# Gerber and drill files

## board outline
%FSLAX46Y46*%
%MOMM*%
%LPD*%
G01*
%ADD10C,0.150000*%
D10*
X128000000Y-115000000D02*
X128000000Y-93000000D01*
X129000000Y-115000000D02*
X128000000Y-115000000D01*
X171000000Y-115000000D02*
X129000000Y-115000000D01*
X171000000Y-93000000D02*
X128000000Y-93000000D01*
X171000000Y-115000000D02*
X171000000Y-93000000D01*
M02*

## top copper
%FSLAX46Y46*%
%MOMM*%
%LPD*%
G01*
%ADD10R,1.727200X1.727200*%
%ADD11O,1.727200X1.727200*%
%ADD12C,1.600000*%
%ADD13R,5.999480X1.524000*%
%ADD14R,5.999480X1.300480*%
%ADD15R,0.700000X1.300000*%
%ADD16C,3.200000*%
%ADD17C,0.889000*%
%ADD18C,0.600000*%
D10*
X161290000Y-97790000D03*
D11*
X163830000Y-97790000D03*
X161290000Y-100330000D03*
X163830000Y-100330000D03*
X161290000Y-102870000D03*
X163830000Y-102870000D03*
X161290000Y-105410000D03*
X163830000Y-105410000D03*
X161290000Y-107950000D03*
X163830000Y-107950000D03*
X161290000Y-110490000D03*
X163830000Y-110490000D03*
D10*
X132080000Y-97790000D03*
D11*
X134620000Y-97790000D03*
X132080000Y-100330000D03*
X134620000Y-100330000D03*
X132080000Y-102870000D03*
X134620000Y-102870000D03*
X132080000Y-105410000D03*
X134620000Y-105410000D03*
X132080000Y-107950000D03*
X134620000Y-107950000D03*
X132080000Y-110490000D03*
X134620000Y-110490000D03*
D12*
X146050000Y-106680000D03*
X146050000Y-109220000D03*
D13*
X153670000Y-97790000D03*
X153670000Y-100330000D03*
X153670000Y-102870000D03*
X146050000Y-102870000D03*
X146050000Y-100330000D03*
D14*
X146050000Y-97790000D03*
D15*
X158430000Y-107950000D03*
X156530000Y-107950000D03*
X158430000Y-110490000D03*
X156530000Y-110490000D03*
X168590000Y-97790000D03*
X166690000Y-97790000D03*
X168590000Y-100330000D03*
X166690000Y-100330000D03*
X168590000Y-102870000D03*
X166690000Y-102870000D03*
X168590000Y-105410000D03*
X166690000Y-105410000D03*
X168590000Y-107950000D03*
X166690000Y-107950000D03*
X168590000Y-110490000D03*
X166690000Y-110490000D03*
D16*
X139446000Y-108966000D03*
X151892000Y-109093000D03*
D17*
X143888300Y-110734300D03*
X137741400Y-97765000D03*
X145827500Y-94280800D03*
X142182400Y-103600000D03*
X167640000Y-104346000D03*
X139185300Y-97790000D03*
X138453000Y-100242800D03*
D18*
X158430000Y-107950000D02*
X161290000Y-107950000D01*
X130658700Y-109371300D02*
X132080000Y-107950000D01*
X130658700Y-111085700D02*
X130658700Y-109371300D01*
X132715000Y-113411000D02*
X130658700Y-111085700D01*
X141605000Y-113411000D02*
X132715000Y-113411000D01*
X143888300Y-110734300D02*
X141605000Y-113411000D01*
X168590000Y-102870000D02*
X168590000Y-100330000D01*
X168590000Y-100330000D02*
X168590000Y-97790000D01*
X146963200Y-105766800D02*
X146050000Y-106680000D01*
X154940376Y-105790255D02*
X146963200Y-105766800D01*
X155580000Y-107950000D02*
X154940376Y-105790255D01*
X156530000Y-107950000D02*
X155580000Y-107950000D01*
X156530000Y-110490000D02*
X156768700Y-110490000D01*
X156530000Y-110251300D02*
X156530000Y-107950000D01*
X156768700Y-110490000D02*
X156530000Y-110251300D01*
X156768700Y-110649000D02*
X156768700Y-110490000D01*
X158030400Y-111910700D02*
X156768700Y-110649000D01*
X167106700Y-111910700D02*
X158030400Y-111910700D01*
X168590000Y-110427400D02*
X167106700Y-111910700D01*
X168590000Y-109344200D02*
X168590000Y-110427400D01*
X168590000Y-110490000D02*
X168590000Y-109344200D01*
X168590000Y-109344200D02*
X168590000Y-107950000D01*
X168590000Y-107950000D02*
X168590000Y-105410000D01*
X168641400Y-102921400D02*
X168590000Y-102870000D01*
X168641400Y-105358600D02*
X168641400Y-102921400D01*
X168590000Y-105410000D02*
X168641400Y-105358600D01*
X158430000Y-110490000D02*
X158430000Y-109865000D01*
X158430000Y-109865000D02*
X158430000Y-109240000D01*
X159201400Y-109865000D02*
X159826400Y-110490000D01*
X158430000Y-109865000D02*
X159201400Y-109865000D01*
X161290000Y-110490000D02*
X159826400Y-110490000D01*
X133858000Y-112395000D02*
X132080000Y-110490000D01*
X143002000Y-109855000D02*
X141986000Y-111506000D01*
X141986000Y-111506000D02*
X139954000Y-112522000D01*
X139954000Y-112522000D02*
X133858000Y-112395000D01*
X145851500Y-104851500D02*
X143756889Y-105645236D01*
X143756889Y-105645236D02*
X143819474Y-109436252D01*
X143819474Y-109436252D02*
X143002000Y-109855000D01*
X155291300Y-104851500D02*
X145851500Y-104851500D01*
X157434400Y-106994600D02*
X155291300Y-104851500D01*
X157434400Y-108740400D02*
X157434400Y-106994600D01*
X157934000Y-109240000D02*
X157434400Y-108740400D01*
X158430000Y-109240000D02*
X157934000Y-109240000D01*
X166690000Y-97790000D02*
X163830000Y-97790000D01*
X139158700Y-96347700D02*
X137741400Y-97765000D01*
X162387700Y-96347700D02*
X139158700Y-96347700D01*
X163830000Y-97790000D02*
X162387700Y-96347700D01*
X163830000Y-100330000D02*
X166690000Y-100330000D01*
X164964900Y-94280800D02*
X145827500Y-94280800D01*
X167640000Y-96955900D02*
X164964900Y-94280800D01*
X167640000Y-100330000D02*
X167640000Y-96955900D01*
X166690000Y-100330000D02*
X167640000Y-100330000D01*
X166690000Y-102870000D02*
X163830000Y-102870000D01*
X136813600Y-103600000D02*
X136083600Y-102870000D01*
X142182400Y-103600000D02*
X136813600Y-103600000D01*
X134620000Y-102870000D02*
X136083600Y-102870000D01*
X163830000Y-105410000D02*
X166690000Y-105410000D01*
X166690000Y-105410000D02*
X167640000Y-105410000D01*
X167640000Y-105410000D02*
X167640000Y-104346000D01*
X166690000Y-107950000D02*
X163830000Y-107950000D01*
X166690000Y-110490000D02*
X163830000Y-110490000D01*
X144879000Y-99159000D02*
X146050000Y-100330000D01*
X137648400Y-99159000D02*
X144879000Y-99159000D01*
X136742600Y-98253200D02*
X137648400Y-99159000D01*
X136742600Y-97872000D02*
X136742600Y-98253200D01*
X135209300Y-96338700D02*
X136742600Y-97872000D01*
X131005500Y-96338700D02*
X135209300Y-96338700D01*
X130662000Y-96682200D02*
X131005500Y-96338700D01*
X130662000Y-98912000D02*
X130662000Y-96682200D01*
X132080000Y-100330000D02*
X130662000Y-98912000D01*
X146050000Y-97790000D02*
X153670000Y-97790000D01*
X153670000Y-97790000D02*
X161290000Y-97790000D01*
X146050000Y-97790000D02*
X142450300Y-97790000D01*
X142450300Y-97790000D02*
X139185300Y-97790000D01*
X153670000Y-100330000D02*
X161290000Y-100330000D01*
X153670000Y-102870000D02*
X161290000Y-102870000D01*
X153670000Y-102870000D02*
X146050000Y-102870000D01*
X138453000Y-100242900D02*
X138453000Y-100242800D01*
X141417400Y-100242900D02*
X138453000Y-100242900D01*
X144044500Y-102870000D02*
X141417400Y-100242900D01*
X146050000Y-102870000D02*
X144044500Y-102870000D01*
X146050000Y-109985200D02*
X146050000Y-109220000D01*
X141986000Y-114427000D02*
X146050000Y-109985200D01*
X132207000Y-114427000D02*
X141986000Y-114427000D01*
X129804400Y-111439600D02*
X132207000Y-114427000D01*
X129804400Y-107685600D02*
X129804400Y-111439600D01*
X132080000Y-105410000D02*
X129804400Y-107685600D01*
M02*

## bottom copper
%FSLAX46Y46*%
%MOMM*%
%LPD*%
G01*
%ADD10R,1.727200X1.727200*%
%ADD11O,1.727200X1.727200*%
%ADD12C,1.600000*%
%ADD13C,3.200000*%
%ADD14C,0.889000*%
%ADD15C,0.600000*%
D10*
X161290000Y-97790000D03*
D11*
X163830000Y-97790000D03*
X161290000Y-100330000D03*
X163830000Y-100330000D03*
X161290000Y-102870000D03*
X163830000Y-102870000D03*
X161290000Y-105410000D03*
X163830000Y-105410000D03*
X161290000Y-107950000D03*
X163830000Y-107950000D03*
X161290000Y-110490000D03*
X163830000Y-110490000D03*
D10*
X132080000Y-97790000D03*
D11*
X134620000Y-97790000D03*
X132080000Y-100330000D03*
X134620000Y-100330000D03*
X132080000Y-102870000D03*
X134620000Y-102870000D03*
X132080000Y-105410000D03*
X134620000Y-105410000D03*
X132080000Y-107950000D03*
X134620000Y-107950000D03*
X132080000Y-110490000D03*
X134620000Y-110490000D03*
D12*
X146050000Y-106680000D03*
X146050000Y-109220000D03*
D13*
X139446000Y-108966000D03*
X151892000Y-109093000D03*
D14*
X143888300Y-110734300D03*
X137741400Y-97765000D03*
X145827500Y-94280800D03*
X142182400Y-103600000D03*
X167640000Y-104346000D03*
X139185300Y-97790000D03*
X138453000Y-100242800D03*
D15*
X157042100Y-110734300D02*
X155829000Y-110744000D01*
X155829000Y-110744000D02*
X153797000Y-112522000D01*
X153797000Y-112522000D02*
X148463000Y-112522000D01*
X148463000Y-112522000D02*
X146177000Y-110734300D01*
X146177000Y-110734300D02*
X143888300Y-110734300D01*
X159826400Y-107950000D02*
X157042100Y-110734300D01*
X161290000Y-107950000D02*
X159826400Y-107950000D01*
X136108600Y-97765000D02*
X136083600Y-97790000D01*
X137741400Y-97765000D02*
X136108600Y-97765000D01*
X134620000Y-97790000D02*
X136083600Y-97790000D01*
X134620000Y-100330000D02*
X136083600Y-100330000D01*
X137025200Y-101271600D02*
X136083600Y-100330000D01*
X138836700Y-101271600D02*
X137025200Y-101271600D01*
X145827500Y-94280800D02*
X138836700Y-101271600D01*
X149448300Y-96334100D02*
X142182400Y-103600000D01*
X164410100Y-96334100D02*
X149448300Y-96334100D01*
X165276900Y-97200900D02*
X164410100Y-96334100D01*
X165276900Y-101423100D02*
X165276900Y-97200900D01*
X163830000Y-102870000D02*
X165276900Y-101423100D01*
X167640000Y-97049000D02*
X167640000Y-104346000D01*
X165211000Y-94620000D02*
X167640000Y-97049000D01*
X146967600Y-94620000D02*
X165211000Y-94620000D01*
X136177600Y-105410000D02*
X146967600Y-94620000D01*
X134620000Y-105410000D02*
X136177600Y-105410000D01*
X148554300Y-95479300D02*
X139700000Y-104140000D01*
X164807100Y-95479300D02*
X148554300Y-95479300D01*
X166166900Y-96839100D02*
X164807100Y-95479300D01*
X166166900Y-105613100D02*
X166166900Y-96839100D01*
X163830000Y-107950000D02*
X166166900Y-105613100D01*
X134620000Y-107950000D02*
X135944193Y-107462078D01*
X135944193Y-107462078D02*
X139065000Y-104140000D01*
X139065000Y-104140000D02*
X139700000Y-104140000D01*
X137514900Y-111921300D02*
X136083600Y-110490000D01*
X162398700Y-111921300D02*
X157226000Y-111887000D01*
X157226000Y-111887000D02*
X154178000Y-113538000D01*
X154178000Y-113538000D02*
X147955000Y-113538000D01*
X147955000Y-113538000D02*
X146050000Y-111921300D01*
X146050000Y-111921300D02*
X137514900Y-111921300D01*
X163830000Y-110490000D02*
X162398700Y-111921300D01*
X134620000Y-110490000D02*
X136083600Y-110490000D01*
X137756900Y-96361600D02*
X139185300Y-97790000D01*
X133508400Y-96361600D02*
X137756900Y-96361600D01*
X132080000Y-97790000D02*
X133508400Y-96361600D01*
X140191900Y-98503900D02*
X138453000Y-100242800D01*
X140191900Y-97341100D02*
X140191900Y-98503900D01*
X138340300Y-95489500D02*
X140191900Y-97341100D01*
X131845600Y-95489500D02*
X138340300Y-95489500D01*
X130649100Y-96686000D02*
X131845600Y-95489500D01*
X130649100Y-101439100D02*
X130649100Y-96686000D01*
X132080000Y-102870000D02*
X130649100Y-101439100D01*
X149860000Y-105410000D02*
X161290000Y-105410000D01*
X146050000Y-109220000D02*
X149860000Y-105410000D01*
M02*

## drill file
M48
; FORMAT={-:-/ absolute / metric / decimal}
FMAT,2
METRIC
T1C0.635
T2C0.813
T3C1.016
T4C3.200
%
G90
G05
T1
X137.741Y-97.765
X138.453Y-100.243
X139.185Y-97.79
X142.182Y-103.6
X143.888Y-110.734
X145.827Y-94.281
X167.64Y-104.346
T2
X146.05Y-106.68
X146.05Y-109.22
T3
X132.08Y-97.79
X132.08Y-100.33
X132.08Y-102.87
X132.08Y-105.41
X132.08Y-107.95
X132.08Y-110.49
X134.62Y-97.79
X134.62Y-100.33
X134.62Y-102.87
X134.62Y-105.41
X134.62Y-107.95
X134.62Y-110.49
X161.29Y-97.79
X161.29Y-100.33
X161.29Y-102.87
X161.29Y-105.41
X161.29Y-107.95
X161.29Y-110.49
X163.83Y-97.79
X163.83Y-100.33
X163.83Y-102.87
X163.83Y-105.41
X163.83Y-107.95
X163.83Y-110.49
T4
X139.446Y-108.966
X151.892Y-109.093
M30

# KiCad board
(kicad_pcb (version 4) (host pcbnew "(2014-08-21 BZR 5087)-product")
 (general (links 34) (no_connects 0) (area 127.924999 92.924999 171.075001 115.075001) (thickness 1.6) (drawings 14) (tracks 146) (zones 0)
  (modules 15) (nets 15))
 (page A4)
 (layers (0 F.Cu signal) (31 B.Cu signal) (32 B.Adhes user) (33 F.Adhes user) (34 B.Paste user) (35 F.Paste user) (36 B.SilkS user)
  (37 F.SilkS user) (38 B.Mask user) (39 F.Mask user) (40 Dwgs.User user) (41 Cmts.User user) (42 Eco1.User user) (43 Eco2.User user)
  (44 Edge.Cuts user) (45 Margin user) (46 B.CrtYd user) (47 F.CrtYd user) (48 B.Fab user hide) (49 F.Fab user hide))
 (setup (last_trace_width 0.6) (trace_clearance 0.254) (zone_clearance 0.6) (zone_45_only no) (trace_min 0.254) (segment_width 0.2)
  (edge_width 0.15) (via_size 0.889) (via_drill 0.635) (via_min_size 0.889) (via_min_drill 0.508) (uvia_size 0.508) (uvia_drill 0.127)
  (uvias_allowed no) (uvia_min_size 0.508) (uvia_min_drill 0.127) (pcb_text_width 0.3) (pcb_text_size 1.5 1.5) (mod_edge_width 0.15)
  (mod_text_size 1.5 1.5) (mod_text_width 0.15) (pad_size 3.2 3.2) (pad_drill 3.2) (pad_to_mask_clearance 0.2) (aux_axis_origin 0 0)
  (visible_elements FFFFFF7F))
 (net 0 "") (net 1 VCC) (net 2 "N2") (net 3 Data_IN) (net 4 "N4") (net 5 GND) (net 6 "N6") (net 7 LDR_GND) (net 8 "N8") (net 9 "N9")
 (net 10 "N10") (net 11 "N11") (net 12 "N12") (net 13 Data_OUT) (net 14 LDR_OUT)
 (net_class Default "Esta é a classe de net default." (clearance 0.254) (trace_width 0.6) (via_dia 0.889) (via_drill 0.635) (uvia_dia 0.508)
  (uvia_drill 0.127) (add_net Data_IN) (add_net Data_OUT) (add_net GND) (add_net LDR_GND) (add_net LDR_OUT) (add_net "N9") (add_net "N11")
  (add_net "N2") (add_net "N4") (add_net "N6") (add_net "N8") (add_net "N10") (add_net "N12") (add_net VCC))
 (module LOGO (layer F.Cu) (at 0 0)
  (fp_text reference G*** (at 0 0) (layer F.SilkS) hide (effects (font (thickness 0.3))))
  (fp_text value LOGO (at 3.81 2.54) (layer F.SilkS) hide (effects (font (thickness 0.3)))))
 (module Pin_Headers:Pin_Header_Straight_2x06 (layer F.Cu) (at 161.29 97.79)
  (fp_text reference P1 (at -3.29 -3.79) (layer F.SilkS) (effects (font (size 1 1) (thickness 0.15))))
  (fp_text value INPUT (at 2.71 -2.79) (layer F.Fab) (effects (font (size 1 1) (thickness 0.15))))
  (pad 1 thru_hole rect (at 0 0) (size 1.7272 1.7272) (drill 1.016) (layers *.Cu *.Mask F.SilkS) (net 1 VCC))
  (pad 2 thru_hole oval (at 2.54 0) (size 1.7272 1.7272) (drill 1.016) (layers *.Cu *.Mask F.SilkS) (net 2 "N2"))
  (pad 3 thru_hole oval (at 0 2.54) (size 1.7272 1.7272) (drill 1.016) (layers *.Cu *.Mask F.SilkS) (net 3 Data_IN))
  (pad 4 thru_hole oval (at 2.54 2.54) (size 1.7272 1.7272) (drill 1.016) (layers *.Cu *.Mask F.SilkS) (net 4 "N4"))
  (pad 5 thru_hole oval (at 0 5.08) (size 1.7272 1.7272) (drill 1.016) (layers *.Cu *.Mask F.SilkS) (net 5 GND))
  (pad 6 thru_hole oval (at 2.54 5.08) (size 1.7272 1.7272) (drill 1.016) (layers *.Cu *.Mask F.SilkS) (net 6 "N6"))
  (pad 7 thru_hole oval (at 0 7.62) (size 1.7272 1.7272) (drill 1.016) (layers *.Cu *.Mask F.SilkS) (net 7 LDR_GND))
  (pad 8 thru_hole oval (at 2.54 7.62) (size 1.7272 1.7272) (drill 1.016) (layers *.Cu *.Mask F.SilkS) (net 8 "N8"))
  (pad 9 thru_hole oval (at 0 10.16) (size 1.7272 1.7272) (drill 1.016) (layers *.Cu *.Mask F.SilkS) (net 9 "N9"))
  (pad 10 thru_hole oval (at 2.54 10.16) (size 1.7272 1.7272) (drill 1.016) (layers *.Cu *.Mask F.SilkS) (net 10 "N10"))
  (pad 11 thru_hole oval (at 0 12.7) (size 1.7272 1.7272) (drill 1.016) (layers *.Cu *.Mask F.SilkS) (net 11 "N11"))
  (pad 12 thru_hole oval (at 2.54 12.7) (size 1.7272 1.7272) (drill 1.016) (layers *.Cu *.Mask F.SilkS) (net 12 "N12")))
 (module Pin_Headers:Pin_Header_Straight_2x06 (layer F.Cu) (at 132.08 97.79)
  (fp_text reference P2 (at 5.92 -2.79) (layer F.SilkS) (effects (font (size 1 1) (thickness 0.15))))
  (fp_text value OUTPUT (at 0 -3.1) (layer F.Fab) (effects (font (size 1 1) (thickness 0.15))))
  (pad 1 thru_hole rect (at 0 0) (size 1.7272 1.7272) (drill 1.016) (layers *.Cu *.Mask F.SilkS) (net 1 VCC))
  (pad 2 thru_hole oval (at 2.54 0) (size 1.7272 1.7272) (drill 1.016) (layers *.Cu *.Mask F.SilkS) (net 2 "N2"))
  (pad 3 thru_hole oval (at 0 2.54) (size 1.7272 1.7272) (drill 1.016) (layers *.Cu *.Mask F.SilkS) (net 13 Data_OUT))
  (pad 4 thru_hole oval (at 2.54 2.54) (size 1.7272 1.7272) (drill 1.016) (layers *.Cu *.Mask F.SilkS) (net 4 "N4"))
  (pad 5 thru_hole oval (at 0 5.08) (size 1.7272 1.7272) (drill 1.016) (layers *.Cu *.Mask F.SilkS) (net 5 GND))
  (pad 6 thru_hole oval (at 2.54 5.08) (size 1.7272 1.7272) (drill 1.016) (layers *.Cu *.Mask F.SilkS) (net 6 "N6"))
  (pad 7 thru_hole oval (at 0 7.62) (size 1.7272 1.7272) (drill 1.016) (layers *.Cu *.Mask F.SilkS) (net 7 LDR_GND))
  (pad 8 thru_hole oval (at 2.54 7.62) (size 1.7272 1.7272) (drill 1.016) (layers *.Cu *.Mask F.SilkS) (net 8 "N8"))
  (pad 9 thru_hole oval (at 0 10.16) (size 1.7272 1.7272) (drill 1.016) (layers *.Cu *.Mask F.SilkS) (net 9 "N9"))
  (pad 10 thru_hole oval (at 2.54 10.16) (size 1.7272 1.7272) (drill 1.016) (layers *.Cu *.Mask F.SilkS) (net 10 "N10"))
  (pad 11 thru_hole oval (at 0 12.7) (size 1.7272 1.7272) (drill 1.016) (layers *.Cu *.Mask F.SilkS) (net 11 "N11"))
  (pad 12 thru_hole oval (at 2.54 12.7) (size 1.7272 1.7272) (drill 1.016) (layers *.Cu *.Mask F.SilkS) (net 12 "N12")))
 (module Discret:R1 (layer F.Cu) (at 146.05 107.95 270)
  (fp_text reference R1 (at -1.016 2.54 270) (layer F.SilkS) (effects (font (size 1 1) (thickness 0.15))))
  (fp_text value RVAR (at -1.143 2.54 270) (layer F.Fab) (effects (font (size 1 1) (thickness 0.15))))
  (pad 1 thru_hole circle (at -1.27 0 270) (size 1.6 1.6) (drill 0.8128) (layers *.Cu *.Mask F.SilkS) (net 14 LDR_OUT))
  (pad 2 thru_hole circle (at 1.27 0 270) (size 1.6 1.6) (drill 0.8128) (layers *.Cu *.Mask F.SilkS) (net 7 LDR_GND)))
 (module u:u (layer F.Cu) (at 149.86 100.33)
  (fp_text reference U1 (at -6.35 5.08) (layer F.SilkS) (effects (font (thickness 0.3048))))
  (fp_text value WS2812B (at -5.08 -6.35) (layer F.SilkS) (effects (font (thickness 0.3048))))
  (pad 1 smd rect (at 3.81 -2.54) (size 5.99948 1.524) (layers F.Cu F.Paste F.Mask) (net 1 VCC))
  (pad 2 smd rect (at 3.81 0) (size 5.99948 1.524) (layers F.Cu F.Paste F.Mask) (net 3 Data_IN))
  (pad 3 smd rect (at 3.81 2.54) (size 5.99948 1.524) (layers F.Cu F.Paste F.Mask) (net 5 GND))
  (pad 4 smd rect (at -3.81 2.54) (size 5.99948 1.524) (layers F.Cu F.Paste F.Mask) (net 5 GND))
  (pad 5 smd rect (at -3.81 0) (size 5.99948 1.524) (layers F.Cu F.Paste F.Mask) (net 13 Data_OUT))
  (pad 6 smd rect (at -3.81 -2.54) (size 5.99948 1.30048) (layers F.Cu F.Paste F.Mask) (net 1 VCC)))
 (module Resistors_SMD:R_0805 (layer F.Cu) (at 157.48 107.95 180)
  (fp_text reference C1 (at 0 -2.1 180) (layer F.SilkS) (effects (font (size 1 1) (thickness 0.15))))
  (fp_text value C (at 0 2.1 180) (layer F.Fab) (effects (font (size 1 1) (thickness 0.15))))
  (pad 1 smd rect (at -0.95 0 180) (size 0.7 1.3) (layers F.Cu F.Paste F.Mask) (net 9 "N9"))
  (pad 2 smd rect (at 0.95 0 180) (size 0.7 1.3) (layers F.Cu F.Paste F.Mask) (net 14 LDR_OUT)))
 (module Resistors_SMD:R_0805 (layer F.Cu) (at 157.48 110.49 180)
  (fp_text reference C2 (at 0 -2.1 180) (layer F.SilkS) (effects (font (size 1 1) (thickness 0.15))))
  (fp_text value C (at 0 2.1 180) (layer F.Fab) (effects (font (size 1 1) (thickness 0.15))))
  (pad 1 smd rect (at -0.95 0 180) (size 0.7 1.3) (layers F.Cu F.Paste F.Mask) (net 11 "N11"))
  (pad 2 smd rect (at 0.95 0 180) (size 0.7 1.3) (layers F.Cu F.Paste F.Mask) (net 14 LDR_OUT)))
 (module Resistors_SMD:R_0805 (layer F.Cu) (at 167.64 97.79 180)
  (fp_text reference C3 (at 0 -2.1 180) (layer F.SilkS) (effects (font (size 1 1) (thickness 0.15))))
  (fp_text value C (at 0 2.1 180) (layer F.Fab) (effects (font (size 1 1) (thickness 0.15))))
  (pad 1 smd rect (at -0.95 0 180) (size 0.7 1.3) (layers F.Cu F.Paste F.Mask) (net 14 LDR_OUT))
  (pad 2 smd rect (at 0.95 0 180) (size 0.7 1.3) (layers F.Cu F.Paste F.Mask) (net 2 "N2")))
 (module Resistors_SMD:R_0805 (layer F.Cu) (at 167.64 100.33 180)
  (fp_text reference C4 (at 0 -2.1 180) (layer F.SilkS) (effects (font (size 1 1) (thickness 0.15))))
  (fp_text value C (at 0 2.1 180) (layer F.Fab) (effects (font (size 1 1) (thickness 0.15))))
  (pad 1 smd rect (at -0.95 0 180) (size 0.7 1.3) (layers F.Cu F.Paste F.Mask) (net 14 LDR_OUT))
  (pad 2 smd rect (at 0.95 0 180) (size 0.7 1.3) (layers F.Cu F.Paste F.Mask) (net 4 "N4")))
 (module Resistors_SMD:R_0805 (layer F.Cu) (at 167.64 102.87 180)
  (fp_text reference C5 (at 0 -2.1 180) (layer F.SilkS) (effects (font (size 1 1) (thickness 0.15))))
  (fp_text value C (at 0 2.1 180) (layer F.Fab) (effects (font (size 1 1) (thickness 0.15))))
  (pad 1 smd rect (at -0.95 0 180) (size 0.7 1.3) (layers F.Cu F.Paste F.Mask) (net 14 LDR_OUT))
  (pad 2 smd rect (at 0.95 0 180) (size 0.7 1.3) (layers F.Cu F.Paste F.Mask) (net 6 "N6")))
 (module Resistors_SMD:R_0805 (layer F.Cu) (at 167.64 105.41 180)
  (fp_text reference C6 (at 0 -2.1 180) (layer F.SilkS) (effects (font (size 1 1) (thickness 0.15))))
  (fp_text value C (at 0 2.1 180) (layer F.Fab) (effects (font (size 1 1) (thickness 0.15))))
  (pad 1 smd rect (at -0.95 0 180) (size 0.7 1.3) (layers F.Cu F.Paste F.Mask) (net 14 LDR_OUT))
  (pad 2 smd rect (at 0.95 0 180) (size 0.7 1.3) (layers F.Cu F.Paste F.Mask) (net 8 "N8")))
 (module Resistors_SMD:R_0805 (layer F.Cu) (at 167.64 107.95 180)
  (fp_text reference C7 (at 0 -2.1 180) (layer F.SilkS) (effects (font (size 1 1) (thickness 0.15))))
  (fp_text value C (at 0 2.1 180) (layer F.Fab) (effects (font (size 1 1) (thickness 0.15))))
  (pad 1 smd rect (at -0.95 0 180) (size 0.7 1.3) (layers F.Cu F.Paste F.Mask) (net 14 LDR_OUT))
  (pad 2 smd rect (at 0.95 0 180) (size 0.7 1.3) (layers F.Cu F.Paste F.Mask) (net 10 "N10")))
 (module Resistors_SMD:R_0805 (layer F.Cu) (at 167.64 110.49 180)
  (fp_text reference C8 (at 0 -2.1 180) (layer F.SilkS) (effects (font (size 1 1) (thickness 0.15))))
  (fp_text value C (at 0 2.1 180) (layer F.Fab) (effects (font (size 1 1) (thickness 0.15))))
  (pad 1 smd rect (at -0.95 0 180) (size 0.7 1.3) (layers F.Cu F.Paste F.Mask) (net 14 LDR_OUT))
  (pad 2 smd rect (at 0.95 0 180) (size 0.7 1.3) (layers F.Cu F.Paste F.Mask) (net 12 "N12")))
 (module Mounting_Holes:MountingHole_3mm (layer F.Cu) (at 139.446 108.966)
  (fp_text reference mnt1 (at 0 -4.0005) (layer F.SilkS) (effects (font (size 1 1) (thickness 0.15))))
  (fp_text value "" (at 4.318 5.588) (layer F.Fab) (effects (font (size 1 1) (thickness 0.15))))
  (pad "" thru_hole circle (at 0 0) (size 3.2 3.2) (drill 3.2) (layers *.Cu *.Mask F.SilkS)))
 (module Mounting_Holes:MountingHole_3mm (layer F.Cu) (at 151.892 109.093)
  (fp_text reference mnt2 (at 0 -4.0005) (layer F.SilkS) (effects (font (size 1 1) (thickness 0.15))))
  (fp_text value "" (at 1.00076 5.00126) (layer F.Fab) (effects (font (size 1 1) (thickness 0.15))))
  (pad "" thru_hole circle (at 0 0) (size 3.2 3.2) (drill 3.2) (layers *.Cu)))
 (gr_line (start 128 115) (end 128 93) (angle 90) (layer Edge.Cuts) (width 0.15))
 (gr_line (start 129 115) (end 128 115) (angle 90) (layer Edge.Cuts) (width 0.15))
 (gr_line (start 171 115) (end 129 115) (angle 90) (layer Edge.Cuts) (width 0.15))
 (gr_line (start 171 93) (end 128 93) (angle 90) (layer Edge.Cuts) (width 0.15))
 (gr_line (start 171 115) (end 171 93) (angle 90) (layer Edge.Cuts) (width 0.15))
 (via (at 143.8883 110.7343) (size 0.889) (layers F.Cu B.Cu) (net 9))
 (segment (start 158.43 107.95) (end 161.29 107.95) (width 0.6) (layer F.Cu) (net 9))
 (segment (start 157.0421 110.7343) (end 155.829 110.744) (width 0.6) (layer B.Cu) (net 9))
 (segment (start 155.829 110.744) (end 153.797 112.522) (width 0.6) (layer B.Cu) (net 9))
 (segment (start 153.797 112.522) (end 148.463 112.522) (width 0.6) (layer B.Cu) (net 9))
 (segment (start 148.463 112.522) (end 146.177 110.7343) (width 0.6) (layer B.Cu) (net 9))
 (segment (start 146.177 110.7343) (end 143.8883 110.7343) (width 0.6) (layer B.Cu) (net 9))
 (segment (start 159.8264 107.95) (end 157.0421 110.7343) (width 0.6) (layer B.Cu) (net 9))
 (segment (start 130.6587 109.3713) (end 132.08 107.95) (width 0.6) (layer F.Cu) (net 9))
 (segment (start 130.6587 111.0857) (end 130.6587 109.3713) (width 0.6) (layer F.Cu) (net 9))
 (segment (start 132.715 113.411) (end 130.6587 111.0857) (width 0.6) (layer F.Cu) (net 9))
 (segment (start 141.605 113.411) (end 132.715 113.411) (width 0.6) (layer F.Cu) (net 9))
 (segment (start 143.8883 110.7343) (end 141.605 113.411) (width 0.6) (layer F.Cu) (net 9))
 (segment (start 161.29 107.95) (end 159.8264 107.95) (width 0.6) (layer B.Cu) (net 9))
 (segment (start 168.59 102.87) (end 168.59 100.33) (width 0.6) (layer F.Cu) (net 14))
 (segment (start 168.59 100.33) (end 168.59 97.79) (width 0.6) (layer F.Cu) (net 14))
 (segment (start 146.9632 105.7668) (end 146.05 106.68) (width 0.6) (layer F.Cu) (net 14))
 (segment (start 154.940376 105.790255) (end 146.9632 105.7668) (width 0.6) (layer F.Cu) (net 14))
 (segment (start 155.58 107.95) (end 154.940376 105.790255) (width 0.6) (layer F.Cu) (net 14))
 (segment (start 156.53 107.95) (end 155.58 107.95) (width 0.6) (layer F.Cu) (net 14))
 (segment (start 156.53 110.49) (end 156.7687 110.49) (width 0.6) (layer F.Cu) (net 14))
 (segment (start 156.53 110.2513) (end 156.53 107.95) (width 0.6) (layer F.Cu) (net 14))
 (segment (start 156.7687 110.49) (end 156.53 110.2513) (width 0.6) (layer F.Cu) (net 14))
 (segment (start 156.7687 110.649) (end 156.7687 110.49) (width 0.6) (layer F.Cu) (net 14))
 (segment (start 158.0304 111.9107) (end 156.7687 110.649) (width 0.6) (layer F.Cu) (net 14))
 (segment (start 167.1067 111.9107) (end 158.0304 111.9107) (width 0.6) (layer F.Cu) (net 14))
 (segment (start 168.59 110.4274) (end 167.1067 111.9107) (width 0.6) (layer F.Cu) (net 14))
 (segment (start 168.59 109.3442) (end 168.59 110.4274) (width 0.6) (layer F.Cu) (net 14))
 (segment (start 168.59 110.49) (end 168.59 109.3442) (width 0.6) (layer F.Cu) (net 14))
 (segment (start 168.59 109.3442) (end 168.59 107.95) (width 0.6) (layer F.Cu) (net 14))
 (segment (start 168.59 107.95) (end 168.59 105.41) (width 0.6) (layer F.Cu) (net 14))
 (segment (start 168.6414 102.9214) (end 168.59 102.87) (width 0.6) (layer F.Cu) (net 14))
 (segment (start 168.6414 105.3586) (end 168.6414 102.9214) (width 0.6) (layer F.Cu) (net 14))
 (segment (start 168.59 105.41) (end 168.6414 105.3586) (width 0.6) (layer F.Cu) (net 14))
 (segment (start 158.43 110.49) (end 158.43 109.865) (width 0.6) (layer F.Cu) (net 11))
 (segment (start 158.43 109.865) (end 158.43 109.24) (width 0.6) (layer F.Cu) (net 11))
 (segment (start 159.2014 109.865) (end 159.8264 110.49) (width 0.6) (layer F.Cu) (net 11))
 (segment (start 158.43 109.865) (end 159.2014 109.865) (width 0.6) (layer F.Cu) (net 11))
 (segment (start 161.29 110.49) (end 159.8264 110.49) (width 0.6) (layer F.Cu) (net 11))
 (segment (start 133.858 112.395) (end 132.08 110.49) (width 0.6) (layer F.Cu) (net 11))
 (segment (start 143.002 109.855) (end 141.986 111.506) (width 0.6) (layer F.Cu) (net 11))
 (segment (start 141.986 111.506) (end 139.954 112.522) (width 0.6) (layer F.Cu) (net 11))
 (segment (start 139.954 112.522) (end 133.858 112.395) (width 0.6) (layer F.Cu) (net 11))
 (segment (start 145.8515 104.8515) (end 143.756889 105.645236) (width 0.6) (layer F.Cu) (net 11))
 (segment (start 143.756889 105.645236) (end 143.819474 109.436252) (width 0.6) (layer F.Cu) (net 11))
 (segment (start 143.819474 109.436252) (end 143.002 109.855) (width 0.6) (layer F.Cu) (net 11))
 (segment (start 155.2913 104.8515) (end 145.8515 104.8515) (width 0.6) (layer F.Cu) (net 11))
 (segment (start 157.4344 106.9946) (end 155.2913 104.8515) (width 0.6) (layer F.Cu) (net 11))
 (segment (start 157.4344 108.7404) (end 157.4344 106.9946) (width 0.6) (layer F.Cu) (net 11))
 (segment (start 157.934 109.24) (end 157.4344 108.7404) (width 0.6) (layer F.Cu) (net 11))
 (segment (start 158.43 109.24) (end 157.934 109.24) (width 0.6) (layer F.Cu) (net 11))
 (via (at 137.7414 97.765) (size 0.889) (layers F.Cu B.Cu) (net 2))
 (segment (start 136.1086 97.765) (end 136.0836 97.79) (width 0.6) (layer B.Cu) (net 2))
 (segment (start 137.7414 97.765) (end 136.1086 97.765) (width 0.6) (layer B.Cu) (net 2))
 (segment (start 134.62 97.79) (end 136.0836 97.79) (width 0.6) (layer B.Cu) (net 2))
 (segment (start 166.69 97.79) (end 163.83 97.79) (width 0.6) (layer F.Cu) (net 2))
 (segment (start 139.1587 96.3477) (end 137.7414 97.765) (width 0.6) (layer F.Cu) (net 2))
 (segment (start 162.3877 96.3477) (end 139.1587 96.3477) (width 0.6) (layer F.Cu) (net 2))
 (segment (start 163.83 97.79) (end 162.3877 96.3477) (width 0.6) (layer F.Cu) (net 2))
 (via (at 145.8275 94.2808) (size 0.889) (layers F.Cu B.Cu) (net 4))
 (segment (start 163.83 100.33) (end 166.69 100.33) (width 0.6) (layer F.Cu) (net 4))
 (segment (start 164.9649 94.2808) (end 145.8275 94.2808) (width 0.6) (layer F.Cu) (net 4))
 (segment (start 167.64 96.9559) (end 164.9649 94.2808) (width 0.6) (layer F.Cu) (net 4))
 (segment (start 167.64 100.33) (end 167.64 96.9559) (width 0.6) (layer F.Cu) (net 4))
 (segment (start 166.69 100.33) (end 167.64 100.33) (width 0.6) (layer F.Cu) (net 4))
 (segment (start 134.62 100.33) (end 136.0836 100.33) (width 0.6) (layer B.Cu) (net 4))
 (segment (start 137.0252 101.2716) (end 136.0836 100.33) (width 0.6) (layer B.Cu) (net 4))
 (segment (start 138.8367 101.2716) (end 137.0252 101.2716) (width 0.6) (layer B.Cu) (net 4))
 (segment (start 145.8275 94.2808) (end 138.8367 101.2716) (width 0.6) (layer B.Cu) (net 4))
 (via (at 142.1824 103.6) (size 0.889) (layers F.Cu B.Cu) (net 6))
 (segment (start 166.69 102.87) (end 163.83 102.87) (width 0.6) (layer F.Cu) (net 6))
 (segment (start 149.4483 96.3341) (end 142.1824 103.6) (width 0.6) (layer B.Cu) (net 6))
 (segment (start 164.4101 96.3341) (end 149.4483 96.3341) (width 0.6) (layer B.Cu) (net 6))
 (segment (start 165.2769 97.2009) (end 164.4101 96.3341) (width 0.6) (layer B.Cu) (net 6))
 (segment (start 165.2769 101.4231) (end 165.2769 97.2009) (width 0.6) (layer B.Cu) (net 6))
 (segment (start 163.83 102.87) (end 165.2769 101.4231) (width 0.6) (layer B.Cu) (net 6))
 (segment (start 136.8136 103.6) (end 136.0836 102.87) (width 0.6) (layer F.Cu) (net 6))
 (segment (start 142.1824 103.6) (end 136.8136 103.6) (width 0.6) (layer F.Cu) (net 6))
 (segment (start 134.62 102.87) (end 136.0836 102.87) (width 0.6) (layer F.Cu) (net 6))
 (via (at 167.64 104.346) (size 0.889) (layers F.Cu B.Cu) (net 8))
 (segment (start 163.83 105.41) (end 166.69 105.41) (width 0.6) (layer F.Cu) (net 8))
 (segment (start 166.69 105.41) (end 167.64 105.41) (width 0.6) (layer F.Cu) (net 8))
 (segment (start 167.64 97.049) (end 167.64 104.346) (width 0.6) (layer B.Cu) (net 8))
 (segment (start 165.211 94.62) (end 167.64 97.049) (width 0.6) (layer B.Cu) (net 8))
 (segment (start 146.9676 94.62) (end 165.211 94.62) (width 0.6) (layer B.Cu) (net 8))
 (segment (start 136.1776 105.41) (end 146.9676 94.62) (width 0.6) (layer B.Cu) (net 8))
 (segment (start 134.62 105.41) (end 136.1776 105.41) (width 0.6) (layer B.Cu) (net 8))
 (segment (start 167.64 105.41) (end 167.64 104.346) (width 0.6) (layer F.Cu) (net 8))
 (segment (start 166.69 107.95) (end 163.83 107.95) (width 0.6) (layer F.Cu) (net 10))
 (segment (start 148.5543 95.4793) (end 139.7 104.14) (width 0.6) (layer B.Cu) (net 10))
 (segment (start 164.8071 95.4793) (end 148.5543 95.4793) (width 0.6) (layer B.Cu) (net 10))
 (segment (start 166.1669 96.8391) (end 164.8071 95.4793) (width 0.6) (layer B.Cu) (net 10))
 (segment (start 166.1669 105.6131) (end 166.1669 96.8391) (width 0.6) (layer B.Cu) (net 10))
 (segment (start 163.83 107.95) (end 166.1669 105.6131) (width 0.6) (layer B.Cu) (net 10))
 (segment (start 134.62 107.95) (end 135.944193 107.462078) (width 0.6) (layer B.Cu) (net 10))
 (segment (start 135.944193 107.462078) (end 139.065 104.14) (width 0.6) (layer B.Cu) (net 10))
 (segment (start 139.065 104.14) (end 139.7 104.14) (width 0.6) (layer B.Cu) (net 10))
 (segment (start 166.69 110.49) (end 163.83 110.49) (width 0.6) (layer F.Cu) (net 12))
 (segment (start 137.5149 111.9213) (end 136.0836 110.49) (width 0.6) (layer B.Cu) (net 12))
 (segment (start 162.3987 111.9213) (end 157.226 111.887) (width 0.6) (layer B.Cu) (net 12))
 (segment (start 157.226 111.887) (end 154.178 113.538) (width 0.6) (layer B.Cu) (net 12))
 (segment (start 154.178 113.538) (end 147.955 113.538) (width 0.6) (layer B.Cu) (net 12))
 (segment (start 147.955 113.538) (end 146.05 111.9213) (width 0.6) (layer B.Cu) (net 12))
 (segment (start 146.05 111.9213) (end 137.5149 111.9213) (width 0.6) (layer B.Cu) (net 12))
 (segment (start 163.83 110.49) (end 162.3987 111.9213) (width 0.6) (layer B.Cu) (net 12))
 (segment (start 134.62 110.49) (end 136.0836 110.49) (width 0.6) (layer B.Cu) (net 12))
 (segment (start 144.879 99.159) (end 146.05 100.33) (width 0.6) (layer F.Cu) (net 13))
 (segment (start 137.6484 99.159) (end 144.879 99.159) (width 0.6) (layer F.Cu) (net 13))
 (segment (start 136.7426 98.2532) (end 137.6484 99.159) (width 0.6) (layer F.Cu) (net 13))
 (segment (start 136.7426 97.872) (end 136.7426 98.2532) (width 0.6) (layer F.Cu) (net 13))
 (segment (start 135.2093 96.3387) (end 136.7426 97.872) (width 0.6) (layer F.Cu) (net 13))
 (segment (start 131.0055 96.3387) (end 135.2093 96.3387) (width 0.6) (layer F.Cu) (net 13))
 (segment (start 130.662 96.6822) (end 131.0055 96.3387) (width 0.6) (layer F.Cu) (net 13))
 (segment (start 130.662 98.912) (end 130.662 96.6822) (width 0.6) (layer F.Cu) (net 13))
 (segment (start 132.08 100.33) (end 130.662 98.912) (width 0.6) (layer F.Cu) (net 13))
 (via (at 139.1853 97.79) (size 0.889) (layers F.Cu B.Cu) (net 1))
 (segment (start 146.05 97.79) (end 153.67 97.79) (width 0.6) (layer F.Cu) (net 1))
 (segment (start 153.67 97.79) (end 161.29 97.79) (width 0.6) (layer F.Cu) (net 1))
 (segment (start 146.05 97.79) (end 142.4503 97.79) (width 0.6) (layer F.Cu) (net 1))
 (segment (start 137.7569 96.3616) (end 139.1853 97.79) (width 0.6) (layer B.Cu) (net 1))
 (segment (start 133.5084 96.3616) (end 137.7569 96.3616) (width 0.6) (layer B.Cu) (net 1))
 (segment (start 132.08 97.79) (end 133.5084 96.3616) (width 0.6) (layer B.Cu) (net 1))
 (segment (start 142.4503 97.79) (end 139.1853 97.79) (width 0.6) (layer F.Cu) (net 1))
 (segment (start 153.67 100.33) (end 161.29 100.33) (width 0.6) (layer F.Cu) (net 3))
 (via (at 138.453 100.2428) (size 0.889) (layers F.Cu B.Cu) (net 5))
 (segment (start 153.67 102.87) (end 161.29 102.87) (width 0.6) (layer F.Cu) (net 5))
 (segment (start 153.67 102.87) (end 146.05 102.87) (width 0.6) (layer F.Cu) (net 5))
 (segment (start 140.1919 98.5039) (end 138.453 100.2428) (width 0.6) (layer B.Cu) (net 5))
 (segment (start 140.1919 97.3411) (end 140.1919 98.5039) (width 0.6) (layer B.Cu) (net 5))
 (segment (start 138.3403 95.4895) (end 140.1919 97.3411) (width 0.6) (layer B.Cu) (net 5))
 (segment (start 131.8456 95.4895) (end 138.3403 95.4895) (width 0.6) (layer B.Cu) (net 5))
 (segment (start 130.6491 96.686) (end 131.8456 95.4895) (width 0.6) (layer B.Cu) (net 5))
 (segment (start 130.6491 101.4391) (end 130.6491 96.686) (width 0.6) (layer B.Cu) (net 5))
 (segment (start 132.08 102.87) (end 130.6491 101.4391) (width 0.6) (layer B.Cu) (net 5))
 (segment (start 138.453 100.2429) (end 138.453 100.2428) (width 0.6) (layer F.Cu) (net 5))
 (segment (start 141.4174 100.2429) (end 138.453 100.2429) (width 0.6) (layer F.Cu) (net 5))
 (segment (start 144.0445 102.87) (end 141.4174 100.2429) (width 0.6) (layer F.Cu) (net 5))
 (segment (start 146.05 102.87) (end 144.0445 102.87) (width 0.6) (layer F.Cu) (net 5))
 (segment (start 149.86 105.41) (end 161.29 105.41) (width 0.6) (layer B.Cu) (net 7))
 (segment (start 146.05 109.22) (end 149.86 105.41) (width 0.6) (layer B.Cu) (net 7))
 (segment (start 146.05 109.9852) (end 146.05 109.22) (width 0.6) (layer F.Cu) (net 7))
 (segment (start 141.986 114.427) (end 146.05 109.9852) (width 0.6) (layer F.Cu) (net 7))
 (segment (start 132.207 114.427) (end 141.986 114.427) (width 0.6) (layer F.Cu) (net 7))
 (segment (start 129.8044 111.4396) (end 132.207 114.427) (width 0.6) (layer F.Cu) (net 7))
 (segment (start 129.8044 107.6856) (end 129.8044 111.4396) (width 0.6) (layer F.Cu) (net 7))
 (segment (start 132.08 105.41) (end 129.8044 107.6856) (width 0.6) (layer F.Cu) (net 7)))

